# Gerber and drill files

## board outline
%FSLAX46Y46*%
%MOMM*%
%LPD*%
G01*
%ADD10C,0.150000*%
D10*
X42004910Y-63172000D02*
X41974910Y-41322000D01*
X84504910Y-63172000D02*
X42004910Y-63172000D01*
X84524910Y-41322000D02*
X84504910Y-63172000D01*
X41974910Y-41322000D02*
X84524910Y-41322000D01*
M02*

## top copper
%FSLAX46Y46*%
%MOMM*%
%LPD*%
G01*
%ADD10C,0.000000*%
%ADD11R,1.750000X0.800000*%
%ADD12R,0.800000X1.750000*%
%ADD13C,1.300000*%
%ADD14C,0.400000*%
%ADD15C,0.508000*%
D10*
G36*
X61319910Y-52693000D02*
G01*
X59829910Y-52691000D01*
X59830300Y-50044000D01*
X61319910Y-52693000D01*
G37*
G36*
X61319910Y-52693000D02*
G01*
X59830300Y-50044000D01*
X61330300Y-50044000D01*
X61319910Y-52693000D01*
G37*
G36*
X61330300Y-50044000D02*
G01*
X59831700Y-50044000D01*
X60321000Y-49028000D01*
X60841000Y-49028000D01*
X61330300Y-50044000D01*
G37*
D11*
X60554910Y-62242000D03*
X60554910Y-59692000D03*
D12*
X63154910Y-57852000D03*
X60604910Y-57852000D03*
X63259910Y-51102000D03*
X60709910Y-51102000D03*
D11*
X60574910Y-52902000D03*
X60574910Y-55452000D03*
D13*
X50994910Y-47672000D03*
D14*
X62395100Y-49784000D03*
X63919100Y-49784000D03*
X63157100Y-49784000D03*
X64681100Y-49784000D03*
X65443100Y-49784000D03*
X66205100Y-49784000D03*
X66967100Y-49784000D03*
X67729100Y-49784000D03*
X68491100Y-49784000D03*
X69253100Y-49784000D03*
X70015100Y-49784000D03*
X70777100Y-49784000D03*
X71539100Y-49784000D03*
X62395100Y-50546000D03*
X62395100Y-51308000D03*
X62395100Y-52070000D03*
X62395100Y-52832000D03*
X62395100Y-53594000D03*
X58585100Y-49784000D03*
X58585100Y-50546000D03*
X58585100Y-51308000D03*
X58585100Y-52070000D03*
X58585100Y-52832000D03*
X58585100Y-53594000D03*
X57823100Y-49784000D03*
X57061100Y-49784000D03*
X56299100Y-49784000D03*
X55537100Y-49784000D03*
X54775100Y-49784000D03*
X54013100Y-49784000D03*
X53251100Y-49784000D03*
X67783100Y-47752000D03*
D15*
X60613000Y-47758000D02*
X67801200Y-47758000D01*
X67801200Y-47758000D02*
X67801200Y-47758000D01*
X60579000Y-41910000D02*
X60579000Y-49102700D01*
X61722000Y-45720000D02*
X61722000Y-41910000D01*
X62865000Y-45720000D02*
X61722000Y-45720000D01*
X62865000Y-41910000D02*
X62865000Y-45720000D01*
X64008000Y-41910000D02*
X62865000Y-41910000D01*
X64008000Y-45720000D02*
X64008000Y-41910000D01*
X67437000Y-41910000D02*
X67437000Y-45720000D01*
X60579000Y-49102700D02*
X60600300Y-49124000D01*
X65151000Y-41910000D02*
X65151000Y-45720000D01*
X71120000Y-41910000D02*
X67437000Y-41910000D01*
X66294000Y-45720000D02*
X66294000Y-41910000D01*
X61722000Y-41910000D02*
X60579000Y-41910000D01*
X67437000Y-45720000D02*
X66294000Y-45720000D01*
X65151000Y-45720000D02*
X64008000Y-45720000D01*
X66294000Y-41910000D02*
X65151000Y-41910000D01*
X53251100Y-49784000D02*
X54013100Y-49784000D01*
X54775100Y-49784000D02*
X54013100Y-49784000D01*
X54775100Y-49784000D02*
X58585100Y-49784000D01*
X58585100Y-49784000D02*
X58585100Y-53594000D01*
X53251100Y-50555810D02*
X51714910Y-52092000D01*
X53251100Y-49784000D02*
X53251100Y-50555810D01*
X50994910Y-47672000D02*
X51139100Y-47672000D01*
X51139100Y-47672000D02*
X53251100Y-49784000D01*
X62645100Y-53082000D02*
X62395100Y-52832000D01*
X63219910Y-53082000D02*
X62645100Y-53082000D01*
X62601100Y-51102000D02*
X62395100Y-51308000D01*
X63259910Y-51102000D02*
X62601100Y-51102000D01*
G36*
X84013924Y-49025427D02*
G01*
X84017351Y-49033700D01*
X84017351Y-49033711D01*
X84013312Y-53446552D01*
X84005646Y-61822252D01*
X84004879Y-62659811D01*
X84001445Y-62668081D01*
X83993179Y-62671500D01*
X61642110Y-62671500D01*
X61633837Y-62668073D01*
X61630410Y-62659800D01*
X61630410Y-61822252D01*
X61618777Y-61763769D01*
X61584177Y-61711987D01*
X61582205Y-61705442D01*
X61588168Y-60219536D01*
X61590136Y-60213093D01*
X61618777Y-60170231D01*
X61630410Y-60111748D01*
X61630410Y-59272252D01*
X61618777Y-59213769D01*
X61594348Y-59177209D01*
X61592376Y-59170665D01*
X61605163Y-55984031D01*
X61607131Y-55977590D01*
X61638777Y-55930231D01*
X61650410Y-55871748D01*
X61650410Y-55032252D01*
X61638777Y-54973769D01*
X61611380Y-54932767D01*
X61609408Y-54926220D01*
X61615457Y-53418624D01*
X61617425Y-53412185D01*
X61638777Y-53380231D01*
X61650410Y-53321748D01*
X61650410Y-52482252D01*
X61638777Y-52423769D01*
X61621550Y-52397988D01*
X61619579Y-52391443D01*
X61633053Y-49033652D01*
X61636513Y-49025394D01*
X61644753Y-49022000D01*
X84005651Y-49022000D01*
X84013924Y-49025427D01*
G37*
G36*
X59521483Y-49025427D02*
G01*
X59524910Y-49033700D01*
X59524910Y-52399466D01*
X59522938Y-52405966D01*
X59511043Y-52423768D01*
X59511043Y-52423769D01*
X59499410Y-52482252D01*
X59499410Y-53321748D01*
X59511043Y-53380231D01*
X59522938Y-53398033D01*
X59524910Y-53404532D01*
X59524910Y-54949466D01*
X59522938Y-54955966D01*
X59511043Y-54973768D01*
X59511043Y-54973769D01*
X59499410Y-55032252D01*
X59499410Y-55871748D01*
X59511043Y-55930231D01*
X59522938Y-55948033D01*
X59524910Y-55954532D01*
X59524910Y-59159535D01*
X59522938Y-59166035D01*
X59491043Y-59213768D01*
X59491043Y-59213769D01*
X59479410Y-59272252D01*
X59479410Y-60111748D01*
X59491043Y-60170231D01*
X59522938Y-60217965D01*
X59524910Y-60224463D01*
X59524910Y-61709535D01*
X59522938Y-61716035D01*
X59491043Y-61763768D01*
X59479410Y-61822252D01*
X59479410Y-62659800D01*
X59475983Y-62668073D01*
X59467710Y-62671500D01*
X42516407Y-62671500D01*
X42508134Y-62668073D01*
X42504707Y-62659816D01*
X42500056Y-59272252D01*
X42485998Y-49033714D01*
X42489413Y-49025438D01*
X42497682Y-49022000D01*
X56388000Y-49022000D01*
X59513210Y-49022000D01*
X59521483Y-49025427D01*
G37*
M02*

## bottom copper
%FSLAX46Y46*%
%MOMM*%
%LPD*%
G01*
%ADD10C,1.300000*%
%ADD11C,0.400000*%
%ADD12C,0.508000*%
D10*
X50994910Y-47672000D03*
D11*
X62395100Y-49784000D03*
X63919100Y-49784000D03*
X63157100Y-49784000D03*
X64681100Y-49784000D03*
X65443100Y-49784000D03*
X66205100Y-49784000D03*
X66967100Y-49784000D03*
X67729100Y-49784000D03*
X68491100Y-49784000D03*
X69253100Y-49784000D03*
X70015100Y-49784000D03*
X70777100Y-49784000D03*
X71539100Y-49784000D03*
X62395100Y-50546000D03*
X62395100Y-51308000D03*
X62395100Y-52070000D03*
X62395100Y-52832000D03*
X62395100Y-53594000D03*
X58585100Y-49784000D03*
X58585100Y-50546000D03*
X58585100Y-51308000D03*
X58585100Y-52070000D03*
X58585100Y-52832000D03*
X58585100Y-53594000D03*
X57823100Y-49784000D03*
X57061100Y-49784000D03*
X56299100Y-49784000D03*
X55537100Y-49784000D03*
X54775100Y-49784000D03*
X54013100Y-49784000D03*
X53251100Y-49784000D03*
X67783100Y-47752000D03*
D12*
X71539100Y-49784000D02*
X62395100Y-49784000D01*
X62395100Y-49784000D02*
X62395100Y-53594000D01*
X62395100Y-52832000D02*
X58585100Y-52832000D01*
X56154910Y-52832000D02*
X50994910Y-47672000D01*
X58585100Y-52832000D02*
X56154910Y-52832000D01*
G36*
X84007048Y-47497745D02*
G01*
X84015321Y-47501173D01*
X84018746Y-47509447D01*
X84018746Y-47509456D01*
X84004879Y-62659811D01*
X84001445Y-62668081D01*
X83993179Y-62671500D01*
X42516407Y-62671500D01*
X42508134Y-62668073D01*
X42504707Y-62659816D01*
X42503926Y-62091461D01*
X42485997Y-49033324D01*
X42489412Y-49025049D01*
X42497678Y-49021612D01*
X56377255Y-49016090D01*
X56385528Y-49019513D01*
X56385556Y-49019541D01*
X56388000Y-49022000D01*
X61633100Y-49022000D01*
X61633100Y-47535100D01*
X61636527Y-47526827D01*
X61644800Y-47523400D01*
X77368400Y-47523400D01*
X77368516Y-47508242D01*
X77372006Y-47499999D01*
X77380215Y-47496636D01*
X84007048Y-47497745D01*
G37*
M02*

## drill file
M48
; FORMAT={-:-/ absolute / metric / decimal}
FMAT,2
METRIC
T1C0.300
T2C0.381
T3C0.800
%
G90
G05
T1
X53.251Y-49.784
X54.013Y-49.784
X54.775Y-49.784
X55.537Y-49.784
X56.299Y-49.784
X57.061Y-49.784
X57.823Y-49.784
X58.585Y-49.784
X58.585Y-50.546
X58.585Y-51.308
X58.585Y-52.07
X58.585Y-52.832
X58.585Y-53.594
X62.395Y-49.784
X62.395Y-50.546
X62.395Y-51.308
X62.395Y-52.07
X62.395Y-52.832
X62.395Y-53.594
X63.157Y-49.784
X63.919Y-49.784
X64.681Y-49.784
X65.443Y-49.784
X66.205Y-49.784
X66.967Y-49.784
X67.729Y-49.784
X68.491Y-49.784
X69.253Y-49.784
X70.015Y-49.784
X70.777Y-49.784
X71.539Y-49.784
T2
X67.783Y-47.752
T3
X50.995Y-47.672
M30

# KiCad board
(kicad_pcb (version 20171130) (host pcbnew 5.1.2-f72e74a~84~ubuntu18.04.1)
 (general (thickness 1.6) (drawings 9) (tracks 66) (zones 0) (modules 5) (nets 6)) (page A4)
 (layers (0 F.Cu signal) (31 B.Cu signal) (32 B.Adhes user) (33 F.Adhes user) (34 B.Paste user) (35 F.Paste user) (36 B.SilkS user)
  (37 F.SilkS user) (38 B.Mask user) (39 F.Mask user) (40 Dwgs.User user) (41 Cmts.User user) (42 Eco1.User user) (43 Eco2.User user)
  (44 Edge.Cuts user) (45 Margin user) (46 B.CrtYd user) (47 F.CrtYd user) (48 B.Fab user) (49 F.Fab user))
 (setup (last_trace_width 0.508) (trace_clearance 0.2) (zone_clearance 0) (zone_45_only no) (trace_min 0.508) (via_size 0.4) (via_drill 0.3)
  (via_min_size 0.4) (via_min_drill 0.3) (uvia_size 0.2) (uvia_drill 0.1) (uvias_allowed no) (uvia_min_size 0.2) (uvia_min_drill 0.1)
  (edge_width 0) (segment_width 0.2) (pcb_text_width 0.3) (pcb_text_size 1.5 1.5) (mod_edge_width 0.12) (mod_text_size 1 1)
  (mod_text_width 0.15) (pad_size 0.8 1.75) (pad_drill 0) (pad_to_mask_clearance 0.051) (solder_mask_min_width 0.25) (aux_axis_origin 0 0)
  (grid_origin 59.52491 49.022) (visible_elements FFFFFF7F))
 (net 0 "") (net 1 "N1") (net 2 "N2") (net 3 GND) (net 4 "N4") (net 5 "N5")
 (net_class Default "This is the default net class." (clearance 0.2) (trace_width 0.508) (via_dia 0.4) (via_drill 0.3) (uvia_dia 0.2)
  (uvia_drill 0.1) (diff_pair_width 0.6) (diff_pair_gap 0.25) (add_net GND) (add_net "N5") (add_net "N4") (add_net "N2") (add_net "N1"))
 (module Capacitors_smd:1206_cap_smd (layer F.Cu) (at 60.55491 60.967 270)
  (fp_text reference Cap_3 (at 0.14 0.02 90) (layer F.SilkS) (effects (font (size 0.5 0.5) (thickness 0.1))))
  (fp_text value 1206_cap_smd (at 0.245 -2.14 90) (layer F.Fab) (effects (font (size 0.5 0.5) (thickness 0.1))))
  (pad 2 smd rect (at 1.275 0 270) (size 0.8 1.75) (layers F.Cu F.Paste F.Mask) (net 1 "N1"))
  (pad 1 smd rect (at -1.275 0 270) (size 0.8 1.75) (layers F.Cu F.Paste F.Mask) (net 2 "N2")))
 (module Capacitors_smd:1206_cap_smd (layer F.Cu) (at 61.87991 57.852)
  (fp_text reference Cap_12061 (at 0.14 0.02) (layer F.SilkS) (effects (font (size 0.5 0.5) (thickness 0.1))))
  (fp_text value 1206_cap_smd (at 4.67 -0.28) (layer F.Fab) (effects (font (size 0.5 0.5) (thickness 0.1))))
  (pad 2 smd rect (at 1.275 0) (size 0.8 1.75) (layers F.Cu F.Paste F.Mask) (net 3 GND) (zone_connect 2))
  (pad 1 smd rect (at -1.275 0) (size 0.8 1.75) (layers F.Cu F.Paste F.Mask) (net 3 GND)))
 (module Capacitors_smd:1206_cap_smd (layer F.Cu) (at 61.98491 51.102) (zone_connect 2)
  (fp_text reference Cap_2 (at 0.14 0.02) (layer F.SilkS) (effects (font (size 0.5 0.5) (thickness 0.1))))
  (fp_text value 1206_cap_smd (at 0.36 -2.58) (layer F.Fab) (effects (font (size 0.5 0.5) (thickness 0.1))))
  (pad 2 smd rect (at 1.275 0) (size 0.8 1.75) (layers F.Cu F.Paste F.Mask) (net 3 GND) (zone_connect 2))
  (pad 1 smd rect (at -1.275 0) (size 0.8 1.75) (layers F.Cu F.Paste F.Mask) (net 3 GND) (zone_connect 2)))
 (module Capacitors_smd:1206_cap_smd (layer F.Cu) (at 60.57491 54.177 90)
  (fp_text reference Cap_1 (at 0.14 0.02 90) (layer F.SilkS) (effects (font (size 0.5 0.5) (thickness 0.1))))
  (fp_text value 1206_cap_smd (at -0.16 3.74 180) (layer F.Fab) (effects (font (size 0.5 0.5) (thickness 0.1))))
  (pad 2 smd rect (at 1.275 0 90) (size 0.8 1.75) (layers F.Cu F.Paste F.Mask) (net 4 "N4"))
  (pad 1 smd rect (at -1.275 0 90) (size 0.8 1.75) (layers F.Cu F.Paste F.Mask) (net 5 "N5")))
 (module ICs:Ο (layer F.Cu) (at 51.05491 47.622)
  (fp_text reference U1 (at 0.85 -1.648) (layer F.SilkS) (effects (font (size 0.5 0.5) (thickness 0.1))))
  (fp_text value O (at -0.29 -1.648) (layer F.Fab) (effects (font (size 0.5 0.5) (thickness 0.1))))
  (pad 1 thru_hole circle (at -0.06 0.05) (size 1.3 1.3) (drill 0.8) (layers *.Cu *.Mask) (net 3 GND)))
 (gr_line (start 42.00491 63.172) (end 41.97491 41.322) (layer Edge.Cuts) (width 0.15))
 (gr_line (start 84.50491 63.172) (end 42.00491 63.172) (layer Edge.Cuts) (width 0.15))
 (gr_line (start 84.52491 41.322) (end 84.50491 63.172) (layer Edge.Cuts) (width 0.15))
 (gr_line (start 41.97491 41.322) (end 84.52491 41.322) (layer Edge.Cuts) (width 0.15))
 (gr_poly (pts (xy 61.31991 52.693) (xy 59.8303 50.044) (xy 59.82991 52.691)) (layer F.Cu) (width 0))
 (gr_poly (pts (xy 61.3303 50.044) (xy 59.8303 50.044) (xy 61.31991 52.693)) (layer F.Cu) (width 0))
 (gr_poly (pts (xy 60.321 49.028) (xy 59.8317 50.044) (xy 61.3303 50.044) (xy 60.841 49.028)) (layer F.Cu) (width 0))
 (segment (start 60.613 47.758) (end 67.8012 47.758) (width 0.508) (layer F.Cu) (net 3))
 (segment (start 67.8012 47.758) (end 67.8012 47.758) (width 0.508) (layer F.Cu) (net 3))
 (via (at 62.3951 49.784) (size 0.4) (drill 0.3) (layers F.Cu B.Cu) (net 3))
 (via (at 63.9191 49.784) (size 0.4) (drill 0.3) (layers F.Cu B.Cu) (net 3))
 (via (at 63.1571 49.784) (size 0.4) (drill 0.3) (layers F.Cu B.Cu) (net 3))
 (via (at 64.6811 49.784) (size 0.4) (drill 0.3) (layers F.Cu B.Cu) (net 3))
 (via (at 65.4431 49.784) (size 0.4) (drill 0.3) (layers F.Cu B.Cu) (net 3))
 (via (at 66.2051 49.784) (size 0.4) (drill 0.3) (layers F.Cu B.Cu) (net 3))
 (via (at 66.9671 49.784) (size 0.4) (drill 0.3) (layers F.Cu B.Cu) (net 3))
 (via (at 67.7291 49.784) (size 0.4) (drill 0.3) (layers F.Cu B.Cu) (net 3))
 (via (at 68.4911 49.784) (size 0.4) (drill 0.3) (layers F.Cu B.Cu) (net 3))
 (via (at 69.2531 49.784) (size 0.4) (drill 0.3) (layers F.Cu B.Cu) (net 3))
 (via (at 70.0151 49.784) (size 0.4) (drill 0.3) (layers F.Cu B.Cu) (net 3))
 (via (at 70.7771 49.784) (size 0.4) (drill 0.3) (layers F.Cu B.Cu) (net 3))
 (via (at 71.5391 49.784) (size 0.4) (drill 0.3) (layers F.Cu B.Cu) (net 3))
 (via (at 62.3951 50.546) (size 0.4) (drill 0.3) (layers F.Cu B.Cu) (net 3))
 (via (at 62.3951 51.308) (size 0.4) (drill 0.3) (layers F.Cu B.Cu) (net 3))
 (via (at 62.3951 52.07) (size 0.4) (drill 0.3) (layers F.Cu B.Cu) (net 3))
 (via (at 62.3951 52.832) (size 0.4) (drill 0.3) (layers F.Cu B.Cu) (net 3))
 (via (at 62.3951 53.594) (size 0.4) (drill 0.3) (layers F.Cu B.Cu) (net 3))
 (via (at 58.5851 49.784) (size 0.4) (drill 0.3) (layers F.Cu B.Cu) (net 3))
 (via (at 58.5851 50.546) (size 0.4) (drill 0.3) (layers F.Cu B.Cu) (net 3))
 (via (at 58.5851 51.308) (size 0.4) (drill 0.3) (layers F.Cu B.Cu) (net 3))
 (via (at 58.5851 52.07) (size 0.4) (drill 0.3) (layers F.Cu B.Cu) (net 3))
 (via (at 58.5851 52.832) (size 0.4) (drill 0.3) (layers F.Cu B.Cu) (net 3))
 (via (at 58.5851 53.594) (size 0.4) (drill 0.3) (layers F.Cu B.Cu) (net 3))
 (via (at 57.8231 49.784) (size 0.4) (drill 0.3) (layers F.Cu B.Cu) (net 3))
 (via (at 57.0611 49.784) (size 0.4) (drill 0.3) (layers F.Cu B.Cu) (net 3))
 (via (at 56.2991 49.784) (size 0.4) (drill 0.3) (layers F.Cu B.Cu) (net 3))
 (via (at 55.5371 49.784) (size 0.4) (drill 0.3) (layers F.Cu B.Cu) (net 3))
 (via (at 54.7751 49.784) (size 0.4) (drill 0.3) (layers F.Cu B.Cu) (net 3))
 (via (at 54.0131 49.784) (size 0.4) (drill 0.3) (layers F.Cu B.Cu) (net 3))
 (via (at 53.2511 49.784) (size 0.4) (drill 0.3) (layers F.Cu B.Cu) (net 3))
 (via (at 67.7831 47.752) (size 0.4) (drill 0.381) (layers F.Cu B.Cu) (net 3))
 (segment (start 60.579 41.91) (end 60.579 49.1027) (width 0.508) (layer F.Cu) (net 3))
 (segment (start 61.722 45.72) (end 61.722 41.91) (width 0.508) (layer F.Cu) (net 3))
 (segment (start 62.865 45.72) (end 61.722 45.72) (width 0.508) (layer F.Cu) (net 3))
 (segment (start 62.865 41.91) (end 62.865 45.72) (width 0.508) (layer F.Cu) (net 3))
 (segment (start 64.008 41.91) (end 62.865 41.91) (width 0.508) (layer F.Cu) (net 3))
 (segment (start 64.008 45.72) (end 64.008 41.91) (width 0.508) (layer F.Cu) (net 3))
 (segment (start 67.437 41.91) (end 67.437 45.72) (width 0.508) (layer F.Cu) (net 3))
 (segment (start 60.579 49.1027) (end 60.6003 49.124) (width 0.508) (layer F.Cu) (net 3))
 (segment (start 65.151 41.91) (end 65.151 45.72) (width 0.508) (layer F.Cu) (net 3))
 (segment (start 71.12 41.91) (end 67.437 41.91) (width 0.508) (layer F.Cu) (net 3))
 (segment (start 66.294 45.72) (end 66.294 41.91) (width 0.508) (layer F.Cu) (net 3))
 (segment (start 61.722 41.91) (end 60.579 41.91) (width 0.508) (layer F.Cu) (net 3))
 (segment (start 67.437 45.72) (end 66.294 45.72) (width 0.508) (layer F.Cu) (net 3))
 (segment (start 65.151 45.72) (end 64.008 45.72) (width 0.508) (layer F.Cu) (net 3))
 (segment (start 66.294 41.91) (end 65.151 41.91) (width 0.508) (layer F.Cu) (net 3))
 (segment (start 53.2511 49.784) (end 54.0131 49.784) (width 0.508) (layer F.Cu) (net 3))
 (segment (start 54.7751 49.784) (end 54.0131 49.784) (width 0.508) (layer F.Cu) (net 3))
 (segment (start 54.7751 49.784) (end 58.5851 49.784) (width 0.508) (layer F.Cu) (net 3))
 (segment (start 58.5851 49.784) (end 58.5851 53.594) (width 0.508) (layer F.Cu) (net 3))
 (segment (start 71.5391 49.784) (end 62.3951 49.784) (width 0.508) (layer B.Cu) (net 3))
 (segment (start 62.3951 49.784) (end 62.3951 53.594) (width 0.508) (layer B.Cu) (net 3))
 (segment (start 53.2511 50.55581) (end 51.71491 52.092) (width 0.508) (layer F.Cu) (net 3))
 (segment (start 53.2511 49.784) (end 53.2511 50.55581) (width 0.508) (layer F.Cu) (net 3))
 (segment (start 50.99491 47.672) (end 51.1391 47.672) (width 0.508) (layer F.Cu) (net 3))
 (segment (start 51.1391 47.672) (end 53.2511 49.784) (width 0.508) (layer F.Cu) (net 3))
 (segment (start 62.6451 53.082) (end 62.3951 52.832) (width 0.508) (layer F.Cu) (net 3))
 (segment (start 63.21991 53.082) (end 62.6451 53.082) (width 0.508) (layer F.Cu) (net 3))
 (segment (start 62.3951 52.832) (end 58.5851 52.832) (width 0.508) (layer B.Cu) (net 3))
 (segment (start 56.15491 52.832) (end 50.99491 47.672) (width 0.508) (layer B.Cu) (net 3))
 (segment (start 58.5851 52.832) (end 56.15491 52.832) (width 0.508) (layer B.Cu) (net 3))
 (segment (start 62.6011 51.102) (end 62.3951 51.308) (width 0.508) (layer F.Cu) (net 3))
 (segment (start 63.25991 51.102) (end 62.6011 51.102) (width 0.508) (layer F.Cu) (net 3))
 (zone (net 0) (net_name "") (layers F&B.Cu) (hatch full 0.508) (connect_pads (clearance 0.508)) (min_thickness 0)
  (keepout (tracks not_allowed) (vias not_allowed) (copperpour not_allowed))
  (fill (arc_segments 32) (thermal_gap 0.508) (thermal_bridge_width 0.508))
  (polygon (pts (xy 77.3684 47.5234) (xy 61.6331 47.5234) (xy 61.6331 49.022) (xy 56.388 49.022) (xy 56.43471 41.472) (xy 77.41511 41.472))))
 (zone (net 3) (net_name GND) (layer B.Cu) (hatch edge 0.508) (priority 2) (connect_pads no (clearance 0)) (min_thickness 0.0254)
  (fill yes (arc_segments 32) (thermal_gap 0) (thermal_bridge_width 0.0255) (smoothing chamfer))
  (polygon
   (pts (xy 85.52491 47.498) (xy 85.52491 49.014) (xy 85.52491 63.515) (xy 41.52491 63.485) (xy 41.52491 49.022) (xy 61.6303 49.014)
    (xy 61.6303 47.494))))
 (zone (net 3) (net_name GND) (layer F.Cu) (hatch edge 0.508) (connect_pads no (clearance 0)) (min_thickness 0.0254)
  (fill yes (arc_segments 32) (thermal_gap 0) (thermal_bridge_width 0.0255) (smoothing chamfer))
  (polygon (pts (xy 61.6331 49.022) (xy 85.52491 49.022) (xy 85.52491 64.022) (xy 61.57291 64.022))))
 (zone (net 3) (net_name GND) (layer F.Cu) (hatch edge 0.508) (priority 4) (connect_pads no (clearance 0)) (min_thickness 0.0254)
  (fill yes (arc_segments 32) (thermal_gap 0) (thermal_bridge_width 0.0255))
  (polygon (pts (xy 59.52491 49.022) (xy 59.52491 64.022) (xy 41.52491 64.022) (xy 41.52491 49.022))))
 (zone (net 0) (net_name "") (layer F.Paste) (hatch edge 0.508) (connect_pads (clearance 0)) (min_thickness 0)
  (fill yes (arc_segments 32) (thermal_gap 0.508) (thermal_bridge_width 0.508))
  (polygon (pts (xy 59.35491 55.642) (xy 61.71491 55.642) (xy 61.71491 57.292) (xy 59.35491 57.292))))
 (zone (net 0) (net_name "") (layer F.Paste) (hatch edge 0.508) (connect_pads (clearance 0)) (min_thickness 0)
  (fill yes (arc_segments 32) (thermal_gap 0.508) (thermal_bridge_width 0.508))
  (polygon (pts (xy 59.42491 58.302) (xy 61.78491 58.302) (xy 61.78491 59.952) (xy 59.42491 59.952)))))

